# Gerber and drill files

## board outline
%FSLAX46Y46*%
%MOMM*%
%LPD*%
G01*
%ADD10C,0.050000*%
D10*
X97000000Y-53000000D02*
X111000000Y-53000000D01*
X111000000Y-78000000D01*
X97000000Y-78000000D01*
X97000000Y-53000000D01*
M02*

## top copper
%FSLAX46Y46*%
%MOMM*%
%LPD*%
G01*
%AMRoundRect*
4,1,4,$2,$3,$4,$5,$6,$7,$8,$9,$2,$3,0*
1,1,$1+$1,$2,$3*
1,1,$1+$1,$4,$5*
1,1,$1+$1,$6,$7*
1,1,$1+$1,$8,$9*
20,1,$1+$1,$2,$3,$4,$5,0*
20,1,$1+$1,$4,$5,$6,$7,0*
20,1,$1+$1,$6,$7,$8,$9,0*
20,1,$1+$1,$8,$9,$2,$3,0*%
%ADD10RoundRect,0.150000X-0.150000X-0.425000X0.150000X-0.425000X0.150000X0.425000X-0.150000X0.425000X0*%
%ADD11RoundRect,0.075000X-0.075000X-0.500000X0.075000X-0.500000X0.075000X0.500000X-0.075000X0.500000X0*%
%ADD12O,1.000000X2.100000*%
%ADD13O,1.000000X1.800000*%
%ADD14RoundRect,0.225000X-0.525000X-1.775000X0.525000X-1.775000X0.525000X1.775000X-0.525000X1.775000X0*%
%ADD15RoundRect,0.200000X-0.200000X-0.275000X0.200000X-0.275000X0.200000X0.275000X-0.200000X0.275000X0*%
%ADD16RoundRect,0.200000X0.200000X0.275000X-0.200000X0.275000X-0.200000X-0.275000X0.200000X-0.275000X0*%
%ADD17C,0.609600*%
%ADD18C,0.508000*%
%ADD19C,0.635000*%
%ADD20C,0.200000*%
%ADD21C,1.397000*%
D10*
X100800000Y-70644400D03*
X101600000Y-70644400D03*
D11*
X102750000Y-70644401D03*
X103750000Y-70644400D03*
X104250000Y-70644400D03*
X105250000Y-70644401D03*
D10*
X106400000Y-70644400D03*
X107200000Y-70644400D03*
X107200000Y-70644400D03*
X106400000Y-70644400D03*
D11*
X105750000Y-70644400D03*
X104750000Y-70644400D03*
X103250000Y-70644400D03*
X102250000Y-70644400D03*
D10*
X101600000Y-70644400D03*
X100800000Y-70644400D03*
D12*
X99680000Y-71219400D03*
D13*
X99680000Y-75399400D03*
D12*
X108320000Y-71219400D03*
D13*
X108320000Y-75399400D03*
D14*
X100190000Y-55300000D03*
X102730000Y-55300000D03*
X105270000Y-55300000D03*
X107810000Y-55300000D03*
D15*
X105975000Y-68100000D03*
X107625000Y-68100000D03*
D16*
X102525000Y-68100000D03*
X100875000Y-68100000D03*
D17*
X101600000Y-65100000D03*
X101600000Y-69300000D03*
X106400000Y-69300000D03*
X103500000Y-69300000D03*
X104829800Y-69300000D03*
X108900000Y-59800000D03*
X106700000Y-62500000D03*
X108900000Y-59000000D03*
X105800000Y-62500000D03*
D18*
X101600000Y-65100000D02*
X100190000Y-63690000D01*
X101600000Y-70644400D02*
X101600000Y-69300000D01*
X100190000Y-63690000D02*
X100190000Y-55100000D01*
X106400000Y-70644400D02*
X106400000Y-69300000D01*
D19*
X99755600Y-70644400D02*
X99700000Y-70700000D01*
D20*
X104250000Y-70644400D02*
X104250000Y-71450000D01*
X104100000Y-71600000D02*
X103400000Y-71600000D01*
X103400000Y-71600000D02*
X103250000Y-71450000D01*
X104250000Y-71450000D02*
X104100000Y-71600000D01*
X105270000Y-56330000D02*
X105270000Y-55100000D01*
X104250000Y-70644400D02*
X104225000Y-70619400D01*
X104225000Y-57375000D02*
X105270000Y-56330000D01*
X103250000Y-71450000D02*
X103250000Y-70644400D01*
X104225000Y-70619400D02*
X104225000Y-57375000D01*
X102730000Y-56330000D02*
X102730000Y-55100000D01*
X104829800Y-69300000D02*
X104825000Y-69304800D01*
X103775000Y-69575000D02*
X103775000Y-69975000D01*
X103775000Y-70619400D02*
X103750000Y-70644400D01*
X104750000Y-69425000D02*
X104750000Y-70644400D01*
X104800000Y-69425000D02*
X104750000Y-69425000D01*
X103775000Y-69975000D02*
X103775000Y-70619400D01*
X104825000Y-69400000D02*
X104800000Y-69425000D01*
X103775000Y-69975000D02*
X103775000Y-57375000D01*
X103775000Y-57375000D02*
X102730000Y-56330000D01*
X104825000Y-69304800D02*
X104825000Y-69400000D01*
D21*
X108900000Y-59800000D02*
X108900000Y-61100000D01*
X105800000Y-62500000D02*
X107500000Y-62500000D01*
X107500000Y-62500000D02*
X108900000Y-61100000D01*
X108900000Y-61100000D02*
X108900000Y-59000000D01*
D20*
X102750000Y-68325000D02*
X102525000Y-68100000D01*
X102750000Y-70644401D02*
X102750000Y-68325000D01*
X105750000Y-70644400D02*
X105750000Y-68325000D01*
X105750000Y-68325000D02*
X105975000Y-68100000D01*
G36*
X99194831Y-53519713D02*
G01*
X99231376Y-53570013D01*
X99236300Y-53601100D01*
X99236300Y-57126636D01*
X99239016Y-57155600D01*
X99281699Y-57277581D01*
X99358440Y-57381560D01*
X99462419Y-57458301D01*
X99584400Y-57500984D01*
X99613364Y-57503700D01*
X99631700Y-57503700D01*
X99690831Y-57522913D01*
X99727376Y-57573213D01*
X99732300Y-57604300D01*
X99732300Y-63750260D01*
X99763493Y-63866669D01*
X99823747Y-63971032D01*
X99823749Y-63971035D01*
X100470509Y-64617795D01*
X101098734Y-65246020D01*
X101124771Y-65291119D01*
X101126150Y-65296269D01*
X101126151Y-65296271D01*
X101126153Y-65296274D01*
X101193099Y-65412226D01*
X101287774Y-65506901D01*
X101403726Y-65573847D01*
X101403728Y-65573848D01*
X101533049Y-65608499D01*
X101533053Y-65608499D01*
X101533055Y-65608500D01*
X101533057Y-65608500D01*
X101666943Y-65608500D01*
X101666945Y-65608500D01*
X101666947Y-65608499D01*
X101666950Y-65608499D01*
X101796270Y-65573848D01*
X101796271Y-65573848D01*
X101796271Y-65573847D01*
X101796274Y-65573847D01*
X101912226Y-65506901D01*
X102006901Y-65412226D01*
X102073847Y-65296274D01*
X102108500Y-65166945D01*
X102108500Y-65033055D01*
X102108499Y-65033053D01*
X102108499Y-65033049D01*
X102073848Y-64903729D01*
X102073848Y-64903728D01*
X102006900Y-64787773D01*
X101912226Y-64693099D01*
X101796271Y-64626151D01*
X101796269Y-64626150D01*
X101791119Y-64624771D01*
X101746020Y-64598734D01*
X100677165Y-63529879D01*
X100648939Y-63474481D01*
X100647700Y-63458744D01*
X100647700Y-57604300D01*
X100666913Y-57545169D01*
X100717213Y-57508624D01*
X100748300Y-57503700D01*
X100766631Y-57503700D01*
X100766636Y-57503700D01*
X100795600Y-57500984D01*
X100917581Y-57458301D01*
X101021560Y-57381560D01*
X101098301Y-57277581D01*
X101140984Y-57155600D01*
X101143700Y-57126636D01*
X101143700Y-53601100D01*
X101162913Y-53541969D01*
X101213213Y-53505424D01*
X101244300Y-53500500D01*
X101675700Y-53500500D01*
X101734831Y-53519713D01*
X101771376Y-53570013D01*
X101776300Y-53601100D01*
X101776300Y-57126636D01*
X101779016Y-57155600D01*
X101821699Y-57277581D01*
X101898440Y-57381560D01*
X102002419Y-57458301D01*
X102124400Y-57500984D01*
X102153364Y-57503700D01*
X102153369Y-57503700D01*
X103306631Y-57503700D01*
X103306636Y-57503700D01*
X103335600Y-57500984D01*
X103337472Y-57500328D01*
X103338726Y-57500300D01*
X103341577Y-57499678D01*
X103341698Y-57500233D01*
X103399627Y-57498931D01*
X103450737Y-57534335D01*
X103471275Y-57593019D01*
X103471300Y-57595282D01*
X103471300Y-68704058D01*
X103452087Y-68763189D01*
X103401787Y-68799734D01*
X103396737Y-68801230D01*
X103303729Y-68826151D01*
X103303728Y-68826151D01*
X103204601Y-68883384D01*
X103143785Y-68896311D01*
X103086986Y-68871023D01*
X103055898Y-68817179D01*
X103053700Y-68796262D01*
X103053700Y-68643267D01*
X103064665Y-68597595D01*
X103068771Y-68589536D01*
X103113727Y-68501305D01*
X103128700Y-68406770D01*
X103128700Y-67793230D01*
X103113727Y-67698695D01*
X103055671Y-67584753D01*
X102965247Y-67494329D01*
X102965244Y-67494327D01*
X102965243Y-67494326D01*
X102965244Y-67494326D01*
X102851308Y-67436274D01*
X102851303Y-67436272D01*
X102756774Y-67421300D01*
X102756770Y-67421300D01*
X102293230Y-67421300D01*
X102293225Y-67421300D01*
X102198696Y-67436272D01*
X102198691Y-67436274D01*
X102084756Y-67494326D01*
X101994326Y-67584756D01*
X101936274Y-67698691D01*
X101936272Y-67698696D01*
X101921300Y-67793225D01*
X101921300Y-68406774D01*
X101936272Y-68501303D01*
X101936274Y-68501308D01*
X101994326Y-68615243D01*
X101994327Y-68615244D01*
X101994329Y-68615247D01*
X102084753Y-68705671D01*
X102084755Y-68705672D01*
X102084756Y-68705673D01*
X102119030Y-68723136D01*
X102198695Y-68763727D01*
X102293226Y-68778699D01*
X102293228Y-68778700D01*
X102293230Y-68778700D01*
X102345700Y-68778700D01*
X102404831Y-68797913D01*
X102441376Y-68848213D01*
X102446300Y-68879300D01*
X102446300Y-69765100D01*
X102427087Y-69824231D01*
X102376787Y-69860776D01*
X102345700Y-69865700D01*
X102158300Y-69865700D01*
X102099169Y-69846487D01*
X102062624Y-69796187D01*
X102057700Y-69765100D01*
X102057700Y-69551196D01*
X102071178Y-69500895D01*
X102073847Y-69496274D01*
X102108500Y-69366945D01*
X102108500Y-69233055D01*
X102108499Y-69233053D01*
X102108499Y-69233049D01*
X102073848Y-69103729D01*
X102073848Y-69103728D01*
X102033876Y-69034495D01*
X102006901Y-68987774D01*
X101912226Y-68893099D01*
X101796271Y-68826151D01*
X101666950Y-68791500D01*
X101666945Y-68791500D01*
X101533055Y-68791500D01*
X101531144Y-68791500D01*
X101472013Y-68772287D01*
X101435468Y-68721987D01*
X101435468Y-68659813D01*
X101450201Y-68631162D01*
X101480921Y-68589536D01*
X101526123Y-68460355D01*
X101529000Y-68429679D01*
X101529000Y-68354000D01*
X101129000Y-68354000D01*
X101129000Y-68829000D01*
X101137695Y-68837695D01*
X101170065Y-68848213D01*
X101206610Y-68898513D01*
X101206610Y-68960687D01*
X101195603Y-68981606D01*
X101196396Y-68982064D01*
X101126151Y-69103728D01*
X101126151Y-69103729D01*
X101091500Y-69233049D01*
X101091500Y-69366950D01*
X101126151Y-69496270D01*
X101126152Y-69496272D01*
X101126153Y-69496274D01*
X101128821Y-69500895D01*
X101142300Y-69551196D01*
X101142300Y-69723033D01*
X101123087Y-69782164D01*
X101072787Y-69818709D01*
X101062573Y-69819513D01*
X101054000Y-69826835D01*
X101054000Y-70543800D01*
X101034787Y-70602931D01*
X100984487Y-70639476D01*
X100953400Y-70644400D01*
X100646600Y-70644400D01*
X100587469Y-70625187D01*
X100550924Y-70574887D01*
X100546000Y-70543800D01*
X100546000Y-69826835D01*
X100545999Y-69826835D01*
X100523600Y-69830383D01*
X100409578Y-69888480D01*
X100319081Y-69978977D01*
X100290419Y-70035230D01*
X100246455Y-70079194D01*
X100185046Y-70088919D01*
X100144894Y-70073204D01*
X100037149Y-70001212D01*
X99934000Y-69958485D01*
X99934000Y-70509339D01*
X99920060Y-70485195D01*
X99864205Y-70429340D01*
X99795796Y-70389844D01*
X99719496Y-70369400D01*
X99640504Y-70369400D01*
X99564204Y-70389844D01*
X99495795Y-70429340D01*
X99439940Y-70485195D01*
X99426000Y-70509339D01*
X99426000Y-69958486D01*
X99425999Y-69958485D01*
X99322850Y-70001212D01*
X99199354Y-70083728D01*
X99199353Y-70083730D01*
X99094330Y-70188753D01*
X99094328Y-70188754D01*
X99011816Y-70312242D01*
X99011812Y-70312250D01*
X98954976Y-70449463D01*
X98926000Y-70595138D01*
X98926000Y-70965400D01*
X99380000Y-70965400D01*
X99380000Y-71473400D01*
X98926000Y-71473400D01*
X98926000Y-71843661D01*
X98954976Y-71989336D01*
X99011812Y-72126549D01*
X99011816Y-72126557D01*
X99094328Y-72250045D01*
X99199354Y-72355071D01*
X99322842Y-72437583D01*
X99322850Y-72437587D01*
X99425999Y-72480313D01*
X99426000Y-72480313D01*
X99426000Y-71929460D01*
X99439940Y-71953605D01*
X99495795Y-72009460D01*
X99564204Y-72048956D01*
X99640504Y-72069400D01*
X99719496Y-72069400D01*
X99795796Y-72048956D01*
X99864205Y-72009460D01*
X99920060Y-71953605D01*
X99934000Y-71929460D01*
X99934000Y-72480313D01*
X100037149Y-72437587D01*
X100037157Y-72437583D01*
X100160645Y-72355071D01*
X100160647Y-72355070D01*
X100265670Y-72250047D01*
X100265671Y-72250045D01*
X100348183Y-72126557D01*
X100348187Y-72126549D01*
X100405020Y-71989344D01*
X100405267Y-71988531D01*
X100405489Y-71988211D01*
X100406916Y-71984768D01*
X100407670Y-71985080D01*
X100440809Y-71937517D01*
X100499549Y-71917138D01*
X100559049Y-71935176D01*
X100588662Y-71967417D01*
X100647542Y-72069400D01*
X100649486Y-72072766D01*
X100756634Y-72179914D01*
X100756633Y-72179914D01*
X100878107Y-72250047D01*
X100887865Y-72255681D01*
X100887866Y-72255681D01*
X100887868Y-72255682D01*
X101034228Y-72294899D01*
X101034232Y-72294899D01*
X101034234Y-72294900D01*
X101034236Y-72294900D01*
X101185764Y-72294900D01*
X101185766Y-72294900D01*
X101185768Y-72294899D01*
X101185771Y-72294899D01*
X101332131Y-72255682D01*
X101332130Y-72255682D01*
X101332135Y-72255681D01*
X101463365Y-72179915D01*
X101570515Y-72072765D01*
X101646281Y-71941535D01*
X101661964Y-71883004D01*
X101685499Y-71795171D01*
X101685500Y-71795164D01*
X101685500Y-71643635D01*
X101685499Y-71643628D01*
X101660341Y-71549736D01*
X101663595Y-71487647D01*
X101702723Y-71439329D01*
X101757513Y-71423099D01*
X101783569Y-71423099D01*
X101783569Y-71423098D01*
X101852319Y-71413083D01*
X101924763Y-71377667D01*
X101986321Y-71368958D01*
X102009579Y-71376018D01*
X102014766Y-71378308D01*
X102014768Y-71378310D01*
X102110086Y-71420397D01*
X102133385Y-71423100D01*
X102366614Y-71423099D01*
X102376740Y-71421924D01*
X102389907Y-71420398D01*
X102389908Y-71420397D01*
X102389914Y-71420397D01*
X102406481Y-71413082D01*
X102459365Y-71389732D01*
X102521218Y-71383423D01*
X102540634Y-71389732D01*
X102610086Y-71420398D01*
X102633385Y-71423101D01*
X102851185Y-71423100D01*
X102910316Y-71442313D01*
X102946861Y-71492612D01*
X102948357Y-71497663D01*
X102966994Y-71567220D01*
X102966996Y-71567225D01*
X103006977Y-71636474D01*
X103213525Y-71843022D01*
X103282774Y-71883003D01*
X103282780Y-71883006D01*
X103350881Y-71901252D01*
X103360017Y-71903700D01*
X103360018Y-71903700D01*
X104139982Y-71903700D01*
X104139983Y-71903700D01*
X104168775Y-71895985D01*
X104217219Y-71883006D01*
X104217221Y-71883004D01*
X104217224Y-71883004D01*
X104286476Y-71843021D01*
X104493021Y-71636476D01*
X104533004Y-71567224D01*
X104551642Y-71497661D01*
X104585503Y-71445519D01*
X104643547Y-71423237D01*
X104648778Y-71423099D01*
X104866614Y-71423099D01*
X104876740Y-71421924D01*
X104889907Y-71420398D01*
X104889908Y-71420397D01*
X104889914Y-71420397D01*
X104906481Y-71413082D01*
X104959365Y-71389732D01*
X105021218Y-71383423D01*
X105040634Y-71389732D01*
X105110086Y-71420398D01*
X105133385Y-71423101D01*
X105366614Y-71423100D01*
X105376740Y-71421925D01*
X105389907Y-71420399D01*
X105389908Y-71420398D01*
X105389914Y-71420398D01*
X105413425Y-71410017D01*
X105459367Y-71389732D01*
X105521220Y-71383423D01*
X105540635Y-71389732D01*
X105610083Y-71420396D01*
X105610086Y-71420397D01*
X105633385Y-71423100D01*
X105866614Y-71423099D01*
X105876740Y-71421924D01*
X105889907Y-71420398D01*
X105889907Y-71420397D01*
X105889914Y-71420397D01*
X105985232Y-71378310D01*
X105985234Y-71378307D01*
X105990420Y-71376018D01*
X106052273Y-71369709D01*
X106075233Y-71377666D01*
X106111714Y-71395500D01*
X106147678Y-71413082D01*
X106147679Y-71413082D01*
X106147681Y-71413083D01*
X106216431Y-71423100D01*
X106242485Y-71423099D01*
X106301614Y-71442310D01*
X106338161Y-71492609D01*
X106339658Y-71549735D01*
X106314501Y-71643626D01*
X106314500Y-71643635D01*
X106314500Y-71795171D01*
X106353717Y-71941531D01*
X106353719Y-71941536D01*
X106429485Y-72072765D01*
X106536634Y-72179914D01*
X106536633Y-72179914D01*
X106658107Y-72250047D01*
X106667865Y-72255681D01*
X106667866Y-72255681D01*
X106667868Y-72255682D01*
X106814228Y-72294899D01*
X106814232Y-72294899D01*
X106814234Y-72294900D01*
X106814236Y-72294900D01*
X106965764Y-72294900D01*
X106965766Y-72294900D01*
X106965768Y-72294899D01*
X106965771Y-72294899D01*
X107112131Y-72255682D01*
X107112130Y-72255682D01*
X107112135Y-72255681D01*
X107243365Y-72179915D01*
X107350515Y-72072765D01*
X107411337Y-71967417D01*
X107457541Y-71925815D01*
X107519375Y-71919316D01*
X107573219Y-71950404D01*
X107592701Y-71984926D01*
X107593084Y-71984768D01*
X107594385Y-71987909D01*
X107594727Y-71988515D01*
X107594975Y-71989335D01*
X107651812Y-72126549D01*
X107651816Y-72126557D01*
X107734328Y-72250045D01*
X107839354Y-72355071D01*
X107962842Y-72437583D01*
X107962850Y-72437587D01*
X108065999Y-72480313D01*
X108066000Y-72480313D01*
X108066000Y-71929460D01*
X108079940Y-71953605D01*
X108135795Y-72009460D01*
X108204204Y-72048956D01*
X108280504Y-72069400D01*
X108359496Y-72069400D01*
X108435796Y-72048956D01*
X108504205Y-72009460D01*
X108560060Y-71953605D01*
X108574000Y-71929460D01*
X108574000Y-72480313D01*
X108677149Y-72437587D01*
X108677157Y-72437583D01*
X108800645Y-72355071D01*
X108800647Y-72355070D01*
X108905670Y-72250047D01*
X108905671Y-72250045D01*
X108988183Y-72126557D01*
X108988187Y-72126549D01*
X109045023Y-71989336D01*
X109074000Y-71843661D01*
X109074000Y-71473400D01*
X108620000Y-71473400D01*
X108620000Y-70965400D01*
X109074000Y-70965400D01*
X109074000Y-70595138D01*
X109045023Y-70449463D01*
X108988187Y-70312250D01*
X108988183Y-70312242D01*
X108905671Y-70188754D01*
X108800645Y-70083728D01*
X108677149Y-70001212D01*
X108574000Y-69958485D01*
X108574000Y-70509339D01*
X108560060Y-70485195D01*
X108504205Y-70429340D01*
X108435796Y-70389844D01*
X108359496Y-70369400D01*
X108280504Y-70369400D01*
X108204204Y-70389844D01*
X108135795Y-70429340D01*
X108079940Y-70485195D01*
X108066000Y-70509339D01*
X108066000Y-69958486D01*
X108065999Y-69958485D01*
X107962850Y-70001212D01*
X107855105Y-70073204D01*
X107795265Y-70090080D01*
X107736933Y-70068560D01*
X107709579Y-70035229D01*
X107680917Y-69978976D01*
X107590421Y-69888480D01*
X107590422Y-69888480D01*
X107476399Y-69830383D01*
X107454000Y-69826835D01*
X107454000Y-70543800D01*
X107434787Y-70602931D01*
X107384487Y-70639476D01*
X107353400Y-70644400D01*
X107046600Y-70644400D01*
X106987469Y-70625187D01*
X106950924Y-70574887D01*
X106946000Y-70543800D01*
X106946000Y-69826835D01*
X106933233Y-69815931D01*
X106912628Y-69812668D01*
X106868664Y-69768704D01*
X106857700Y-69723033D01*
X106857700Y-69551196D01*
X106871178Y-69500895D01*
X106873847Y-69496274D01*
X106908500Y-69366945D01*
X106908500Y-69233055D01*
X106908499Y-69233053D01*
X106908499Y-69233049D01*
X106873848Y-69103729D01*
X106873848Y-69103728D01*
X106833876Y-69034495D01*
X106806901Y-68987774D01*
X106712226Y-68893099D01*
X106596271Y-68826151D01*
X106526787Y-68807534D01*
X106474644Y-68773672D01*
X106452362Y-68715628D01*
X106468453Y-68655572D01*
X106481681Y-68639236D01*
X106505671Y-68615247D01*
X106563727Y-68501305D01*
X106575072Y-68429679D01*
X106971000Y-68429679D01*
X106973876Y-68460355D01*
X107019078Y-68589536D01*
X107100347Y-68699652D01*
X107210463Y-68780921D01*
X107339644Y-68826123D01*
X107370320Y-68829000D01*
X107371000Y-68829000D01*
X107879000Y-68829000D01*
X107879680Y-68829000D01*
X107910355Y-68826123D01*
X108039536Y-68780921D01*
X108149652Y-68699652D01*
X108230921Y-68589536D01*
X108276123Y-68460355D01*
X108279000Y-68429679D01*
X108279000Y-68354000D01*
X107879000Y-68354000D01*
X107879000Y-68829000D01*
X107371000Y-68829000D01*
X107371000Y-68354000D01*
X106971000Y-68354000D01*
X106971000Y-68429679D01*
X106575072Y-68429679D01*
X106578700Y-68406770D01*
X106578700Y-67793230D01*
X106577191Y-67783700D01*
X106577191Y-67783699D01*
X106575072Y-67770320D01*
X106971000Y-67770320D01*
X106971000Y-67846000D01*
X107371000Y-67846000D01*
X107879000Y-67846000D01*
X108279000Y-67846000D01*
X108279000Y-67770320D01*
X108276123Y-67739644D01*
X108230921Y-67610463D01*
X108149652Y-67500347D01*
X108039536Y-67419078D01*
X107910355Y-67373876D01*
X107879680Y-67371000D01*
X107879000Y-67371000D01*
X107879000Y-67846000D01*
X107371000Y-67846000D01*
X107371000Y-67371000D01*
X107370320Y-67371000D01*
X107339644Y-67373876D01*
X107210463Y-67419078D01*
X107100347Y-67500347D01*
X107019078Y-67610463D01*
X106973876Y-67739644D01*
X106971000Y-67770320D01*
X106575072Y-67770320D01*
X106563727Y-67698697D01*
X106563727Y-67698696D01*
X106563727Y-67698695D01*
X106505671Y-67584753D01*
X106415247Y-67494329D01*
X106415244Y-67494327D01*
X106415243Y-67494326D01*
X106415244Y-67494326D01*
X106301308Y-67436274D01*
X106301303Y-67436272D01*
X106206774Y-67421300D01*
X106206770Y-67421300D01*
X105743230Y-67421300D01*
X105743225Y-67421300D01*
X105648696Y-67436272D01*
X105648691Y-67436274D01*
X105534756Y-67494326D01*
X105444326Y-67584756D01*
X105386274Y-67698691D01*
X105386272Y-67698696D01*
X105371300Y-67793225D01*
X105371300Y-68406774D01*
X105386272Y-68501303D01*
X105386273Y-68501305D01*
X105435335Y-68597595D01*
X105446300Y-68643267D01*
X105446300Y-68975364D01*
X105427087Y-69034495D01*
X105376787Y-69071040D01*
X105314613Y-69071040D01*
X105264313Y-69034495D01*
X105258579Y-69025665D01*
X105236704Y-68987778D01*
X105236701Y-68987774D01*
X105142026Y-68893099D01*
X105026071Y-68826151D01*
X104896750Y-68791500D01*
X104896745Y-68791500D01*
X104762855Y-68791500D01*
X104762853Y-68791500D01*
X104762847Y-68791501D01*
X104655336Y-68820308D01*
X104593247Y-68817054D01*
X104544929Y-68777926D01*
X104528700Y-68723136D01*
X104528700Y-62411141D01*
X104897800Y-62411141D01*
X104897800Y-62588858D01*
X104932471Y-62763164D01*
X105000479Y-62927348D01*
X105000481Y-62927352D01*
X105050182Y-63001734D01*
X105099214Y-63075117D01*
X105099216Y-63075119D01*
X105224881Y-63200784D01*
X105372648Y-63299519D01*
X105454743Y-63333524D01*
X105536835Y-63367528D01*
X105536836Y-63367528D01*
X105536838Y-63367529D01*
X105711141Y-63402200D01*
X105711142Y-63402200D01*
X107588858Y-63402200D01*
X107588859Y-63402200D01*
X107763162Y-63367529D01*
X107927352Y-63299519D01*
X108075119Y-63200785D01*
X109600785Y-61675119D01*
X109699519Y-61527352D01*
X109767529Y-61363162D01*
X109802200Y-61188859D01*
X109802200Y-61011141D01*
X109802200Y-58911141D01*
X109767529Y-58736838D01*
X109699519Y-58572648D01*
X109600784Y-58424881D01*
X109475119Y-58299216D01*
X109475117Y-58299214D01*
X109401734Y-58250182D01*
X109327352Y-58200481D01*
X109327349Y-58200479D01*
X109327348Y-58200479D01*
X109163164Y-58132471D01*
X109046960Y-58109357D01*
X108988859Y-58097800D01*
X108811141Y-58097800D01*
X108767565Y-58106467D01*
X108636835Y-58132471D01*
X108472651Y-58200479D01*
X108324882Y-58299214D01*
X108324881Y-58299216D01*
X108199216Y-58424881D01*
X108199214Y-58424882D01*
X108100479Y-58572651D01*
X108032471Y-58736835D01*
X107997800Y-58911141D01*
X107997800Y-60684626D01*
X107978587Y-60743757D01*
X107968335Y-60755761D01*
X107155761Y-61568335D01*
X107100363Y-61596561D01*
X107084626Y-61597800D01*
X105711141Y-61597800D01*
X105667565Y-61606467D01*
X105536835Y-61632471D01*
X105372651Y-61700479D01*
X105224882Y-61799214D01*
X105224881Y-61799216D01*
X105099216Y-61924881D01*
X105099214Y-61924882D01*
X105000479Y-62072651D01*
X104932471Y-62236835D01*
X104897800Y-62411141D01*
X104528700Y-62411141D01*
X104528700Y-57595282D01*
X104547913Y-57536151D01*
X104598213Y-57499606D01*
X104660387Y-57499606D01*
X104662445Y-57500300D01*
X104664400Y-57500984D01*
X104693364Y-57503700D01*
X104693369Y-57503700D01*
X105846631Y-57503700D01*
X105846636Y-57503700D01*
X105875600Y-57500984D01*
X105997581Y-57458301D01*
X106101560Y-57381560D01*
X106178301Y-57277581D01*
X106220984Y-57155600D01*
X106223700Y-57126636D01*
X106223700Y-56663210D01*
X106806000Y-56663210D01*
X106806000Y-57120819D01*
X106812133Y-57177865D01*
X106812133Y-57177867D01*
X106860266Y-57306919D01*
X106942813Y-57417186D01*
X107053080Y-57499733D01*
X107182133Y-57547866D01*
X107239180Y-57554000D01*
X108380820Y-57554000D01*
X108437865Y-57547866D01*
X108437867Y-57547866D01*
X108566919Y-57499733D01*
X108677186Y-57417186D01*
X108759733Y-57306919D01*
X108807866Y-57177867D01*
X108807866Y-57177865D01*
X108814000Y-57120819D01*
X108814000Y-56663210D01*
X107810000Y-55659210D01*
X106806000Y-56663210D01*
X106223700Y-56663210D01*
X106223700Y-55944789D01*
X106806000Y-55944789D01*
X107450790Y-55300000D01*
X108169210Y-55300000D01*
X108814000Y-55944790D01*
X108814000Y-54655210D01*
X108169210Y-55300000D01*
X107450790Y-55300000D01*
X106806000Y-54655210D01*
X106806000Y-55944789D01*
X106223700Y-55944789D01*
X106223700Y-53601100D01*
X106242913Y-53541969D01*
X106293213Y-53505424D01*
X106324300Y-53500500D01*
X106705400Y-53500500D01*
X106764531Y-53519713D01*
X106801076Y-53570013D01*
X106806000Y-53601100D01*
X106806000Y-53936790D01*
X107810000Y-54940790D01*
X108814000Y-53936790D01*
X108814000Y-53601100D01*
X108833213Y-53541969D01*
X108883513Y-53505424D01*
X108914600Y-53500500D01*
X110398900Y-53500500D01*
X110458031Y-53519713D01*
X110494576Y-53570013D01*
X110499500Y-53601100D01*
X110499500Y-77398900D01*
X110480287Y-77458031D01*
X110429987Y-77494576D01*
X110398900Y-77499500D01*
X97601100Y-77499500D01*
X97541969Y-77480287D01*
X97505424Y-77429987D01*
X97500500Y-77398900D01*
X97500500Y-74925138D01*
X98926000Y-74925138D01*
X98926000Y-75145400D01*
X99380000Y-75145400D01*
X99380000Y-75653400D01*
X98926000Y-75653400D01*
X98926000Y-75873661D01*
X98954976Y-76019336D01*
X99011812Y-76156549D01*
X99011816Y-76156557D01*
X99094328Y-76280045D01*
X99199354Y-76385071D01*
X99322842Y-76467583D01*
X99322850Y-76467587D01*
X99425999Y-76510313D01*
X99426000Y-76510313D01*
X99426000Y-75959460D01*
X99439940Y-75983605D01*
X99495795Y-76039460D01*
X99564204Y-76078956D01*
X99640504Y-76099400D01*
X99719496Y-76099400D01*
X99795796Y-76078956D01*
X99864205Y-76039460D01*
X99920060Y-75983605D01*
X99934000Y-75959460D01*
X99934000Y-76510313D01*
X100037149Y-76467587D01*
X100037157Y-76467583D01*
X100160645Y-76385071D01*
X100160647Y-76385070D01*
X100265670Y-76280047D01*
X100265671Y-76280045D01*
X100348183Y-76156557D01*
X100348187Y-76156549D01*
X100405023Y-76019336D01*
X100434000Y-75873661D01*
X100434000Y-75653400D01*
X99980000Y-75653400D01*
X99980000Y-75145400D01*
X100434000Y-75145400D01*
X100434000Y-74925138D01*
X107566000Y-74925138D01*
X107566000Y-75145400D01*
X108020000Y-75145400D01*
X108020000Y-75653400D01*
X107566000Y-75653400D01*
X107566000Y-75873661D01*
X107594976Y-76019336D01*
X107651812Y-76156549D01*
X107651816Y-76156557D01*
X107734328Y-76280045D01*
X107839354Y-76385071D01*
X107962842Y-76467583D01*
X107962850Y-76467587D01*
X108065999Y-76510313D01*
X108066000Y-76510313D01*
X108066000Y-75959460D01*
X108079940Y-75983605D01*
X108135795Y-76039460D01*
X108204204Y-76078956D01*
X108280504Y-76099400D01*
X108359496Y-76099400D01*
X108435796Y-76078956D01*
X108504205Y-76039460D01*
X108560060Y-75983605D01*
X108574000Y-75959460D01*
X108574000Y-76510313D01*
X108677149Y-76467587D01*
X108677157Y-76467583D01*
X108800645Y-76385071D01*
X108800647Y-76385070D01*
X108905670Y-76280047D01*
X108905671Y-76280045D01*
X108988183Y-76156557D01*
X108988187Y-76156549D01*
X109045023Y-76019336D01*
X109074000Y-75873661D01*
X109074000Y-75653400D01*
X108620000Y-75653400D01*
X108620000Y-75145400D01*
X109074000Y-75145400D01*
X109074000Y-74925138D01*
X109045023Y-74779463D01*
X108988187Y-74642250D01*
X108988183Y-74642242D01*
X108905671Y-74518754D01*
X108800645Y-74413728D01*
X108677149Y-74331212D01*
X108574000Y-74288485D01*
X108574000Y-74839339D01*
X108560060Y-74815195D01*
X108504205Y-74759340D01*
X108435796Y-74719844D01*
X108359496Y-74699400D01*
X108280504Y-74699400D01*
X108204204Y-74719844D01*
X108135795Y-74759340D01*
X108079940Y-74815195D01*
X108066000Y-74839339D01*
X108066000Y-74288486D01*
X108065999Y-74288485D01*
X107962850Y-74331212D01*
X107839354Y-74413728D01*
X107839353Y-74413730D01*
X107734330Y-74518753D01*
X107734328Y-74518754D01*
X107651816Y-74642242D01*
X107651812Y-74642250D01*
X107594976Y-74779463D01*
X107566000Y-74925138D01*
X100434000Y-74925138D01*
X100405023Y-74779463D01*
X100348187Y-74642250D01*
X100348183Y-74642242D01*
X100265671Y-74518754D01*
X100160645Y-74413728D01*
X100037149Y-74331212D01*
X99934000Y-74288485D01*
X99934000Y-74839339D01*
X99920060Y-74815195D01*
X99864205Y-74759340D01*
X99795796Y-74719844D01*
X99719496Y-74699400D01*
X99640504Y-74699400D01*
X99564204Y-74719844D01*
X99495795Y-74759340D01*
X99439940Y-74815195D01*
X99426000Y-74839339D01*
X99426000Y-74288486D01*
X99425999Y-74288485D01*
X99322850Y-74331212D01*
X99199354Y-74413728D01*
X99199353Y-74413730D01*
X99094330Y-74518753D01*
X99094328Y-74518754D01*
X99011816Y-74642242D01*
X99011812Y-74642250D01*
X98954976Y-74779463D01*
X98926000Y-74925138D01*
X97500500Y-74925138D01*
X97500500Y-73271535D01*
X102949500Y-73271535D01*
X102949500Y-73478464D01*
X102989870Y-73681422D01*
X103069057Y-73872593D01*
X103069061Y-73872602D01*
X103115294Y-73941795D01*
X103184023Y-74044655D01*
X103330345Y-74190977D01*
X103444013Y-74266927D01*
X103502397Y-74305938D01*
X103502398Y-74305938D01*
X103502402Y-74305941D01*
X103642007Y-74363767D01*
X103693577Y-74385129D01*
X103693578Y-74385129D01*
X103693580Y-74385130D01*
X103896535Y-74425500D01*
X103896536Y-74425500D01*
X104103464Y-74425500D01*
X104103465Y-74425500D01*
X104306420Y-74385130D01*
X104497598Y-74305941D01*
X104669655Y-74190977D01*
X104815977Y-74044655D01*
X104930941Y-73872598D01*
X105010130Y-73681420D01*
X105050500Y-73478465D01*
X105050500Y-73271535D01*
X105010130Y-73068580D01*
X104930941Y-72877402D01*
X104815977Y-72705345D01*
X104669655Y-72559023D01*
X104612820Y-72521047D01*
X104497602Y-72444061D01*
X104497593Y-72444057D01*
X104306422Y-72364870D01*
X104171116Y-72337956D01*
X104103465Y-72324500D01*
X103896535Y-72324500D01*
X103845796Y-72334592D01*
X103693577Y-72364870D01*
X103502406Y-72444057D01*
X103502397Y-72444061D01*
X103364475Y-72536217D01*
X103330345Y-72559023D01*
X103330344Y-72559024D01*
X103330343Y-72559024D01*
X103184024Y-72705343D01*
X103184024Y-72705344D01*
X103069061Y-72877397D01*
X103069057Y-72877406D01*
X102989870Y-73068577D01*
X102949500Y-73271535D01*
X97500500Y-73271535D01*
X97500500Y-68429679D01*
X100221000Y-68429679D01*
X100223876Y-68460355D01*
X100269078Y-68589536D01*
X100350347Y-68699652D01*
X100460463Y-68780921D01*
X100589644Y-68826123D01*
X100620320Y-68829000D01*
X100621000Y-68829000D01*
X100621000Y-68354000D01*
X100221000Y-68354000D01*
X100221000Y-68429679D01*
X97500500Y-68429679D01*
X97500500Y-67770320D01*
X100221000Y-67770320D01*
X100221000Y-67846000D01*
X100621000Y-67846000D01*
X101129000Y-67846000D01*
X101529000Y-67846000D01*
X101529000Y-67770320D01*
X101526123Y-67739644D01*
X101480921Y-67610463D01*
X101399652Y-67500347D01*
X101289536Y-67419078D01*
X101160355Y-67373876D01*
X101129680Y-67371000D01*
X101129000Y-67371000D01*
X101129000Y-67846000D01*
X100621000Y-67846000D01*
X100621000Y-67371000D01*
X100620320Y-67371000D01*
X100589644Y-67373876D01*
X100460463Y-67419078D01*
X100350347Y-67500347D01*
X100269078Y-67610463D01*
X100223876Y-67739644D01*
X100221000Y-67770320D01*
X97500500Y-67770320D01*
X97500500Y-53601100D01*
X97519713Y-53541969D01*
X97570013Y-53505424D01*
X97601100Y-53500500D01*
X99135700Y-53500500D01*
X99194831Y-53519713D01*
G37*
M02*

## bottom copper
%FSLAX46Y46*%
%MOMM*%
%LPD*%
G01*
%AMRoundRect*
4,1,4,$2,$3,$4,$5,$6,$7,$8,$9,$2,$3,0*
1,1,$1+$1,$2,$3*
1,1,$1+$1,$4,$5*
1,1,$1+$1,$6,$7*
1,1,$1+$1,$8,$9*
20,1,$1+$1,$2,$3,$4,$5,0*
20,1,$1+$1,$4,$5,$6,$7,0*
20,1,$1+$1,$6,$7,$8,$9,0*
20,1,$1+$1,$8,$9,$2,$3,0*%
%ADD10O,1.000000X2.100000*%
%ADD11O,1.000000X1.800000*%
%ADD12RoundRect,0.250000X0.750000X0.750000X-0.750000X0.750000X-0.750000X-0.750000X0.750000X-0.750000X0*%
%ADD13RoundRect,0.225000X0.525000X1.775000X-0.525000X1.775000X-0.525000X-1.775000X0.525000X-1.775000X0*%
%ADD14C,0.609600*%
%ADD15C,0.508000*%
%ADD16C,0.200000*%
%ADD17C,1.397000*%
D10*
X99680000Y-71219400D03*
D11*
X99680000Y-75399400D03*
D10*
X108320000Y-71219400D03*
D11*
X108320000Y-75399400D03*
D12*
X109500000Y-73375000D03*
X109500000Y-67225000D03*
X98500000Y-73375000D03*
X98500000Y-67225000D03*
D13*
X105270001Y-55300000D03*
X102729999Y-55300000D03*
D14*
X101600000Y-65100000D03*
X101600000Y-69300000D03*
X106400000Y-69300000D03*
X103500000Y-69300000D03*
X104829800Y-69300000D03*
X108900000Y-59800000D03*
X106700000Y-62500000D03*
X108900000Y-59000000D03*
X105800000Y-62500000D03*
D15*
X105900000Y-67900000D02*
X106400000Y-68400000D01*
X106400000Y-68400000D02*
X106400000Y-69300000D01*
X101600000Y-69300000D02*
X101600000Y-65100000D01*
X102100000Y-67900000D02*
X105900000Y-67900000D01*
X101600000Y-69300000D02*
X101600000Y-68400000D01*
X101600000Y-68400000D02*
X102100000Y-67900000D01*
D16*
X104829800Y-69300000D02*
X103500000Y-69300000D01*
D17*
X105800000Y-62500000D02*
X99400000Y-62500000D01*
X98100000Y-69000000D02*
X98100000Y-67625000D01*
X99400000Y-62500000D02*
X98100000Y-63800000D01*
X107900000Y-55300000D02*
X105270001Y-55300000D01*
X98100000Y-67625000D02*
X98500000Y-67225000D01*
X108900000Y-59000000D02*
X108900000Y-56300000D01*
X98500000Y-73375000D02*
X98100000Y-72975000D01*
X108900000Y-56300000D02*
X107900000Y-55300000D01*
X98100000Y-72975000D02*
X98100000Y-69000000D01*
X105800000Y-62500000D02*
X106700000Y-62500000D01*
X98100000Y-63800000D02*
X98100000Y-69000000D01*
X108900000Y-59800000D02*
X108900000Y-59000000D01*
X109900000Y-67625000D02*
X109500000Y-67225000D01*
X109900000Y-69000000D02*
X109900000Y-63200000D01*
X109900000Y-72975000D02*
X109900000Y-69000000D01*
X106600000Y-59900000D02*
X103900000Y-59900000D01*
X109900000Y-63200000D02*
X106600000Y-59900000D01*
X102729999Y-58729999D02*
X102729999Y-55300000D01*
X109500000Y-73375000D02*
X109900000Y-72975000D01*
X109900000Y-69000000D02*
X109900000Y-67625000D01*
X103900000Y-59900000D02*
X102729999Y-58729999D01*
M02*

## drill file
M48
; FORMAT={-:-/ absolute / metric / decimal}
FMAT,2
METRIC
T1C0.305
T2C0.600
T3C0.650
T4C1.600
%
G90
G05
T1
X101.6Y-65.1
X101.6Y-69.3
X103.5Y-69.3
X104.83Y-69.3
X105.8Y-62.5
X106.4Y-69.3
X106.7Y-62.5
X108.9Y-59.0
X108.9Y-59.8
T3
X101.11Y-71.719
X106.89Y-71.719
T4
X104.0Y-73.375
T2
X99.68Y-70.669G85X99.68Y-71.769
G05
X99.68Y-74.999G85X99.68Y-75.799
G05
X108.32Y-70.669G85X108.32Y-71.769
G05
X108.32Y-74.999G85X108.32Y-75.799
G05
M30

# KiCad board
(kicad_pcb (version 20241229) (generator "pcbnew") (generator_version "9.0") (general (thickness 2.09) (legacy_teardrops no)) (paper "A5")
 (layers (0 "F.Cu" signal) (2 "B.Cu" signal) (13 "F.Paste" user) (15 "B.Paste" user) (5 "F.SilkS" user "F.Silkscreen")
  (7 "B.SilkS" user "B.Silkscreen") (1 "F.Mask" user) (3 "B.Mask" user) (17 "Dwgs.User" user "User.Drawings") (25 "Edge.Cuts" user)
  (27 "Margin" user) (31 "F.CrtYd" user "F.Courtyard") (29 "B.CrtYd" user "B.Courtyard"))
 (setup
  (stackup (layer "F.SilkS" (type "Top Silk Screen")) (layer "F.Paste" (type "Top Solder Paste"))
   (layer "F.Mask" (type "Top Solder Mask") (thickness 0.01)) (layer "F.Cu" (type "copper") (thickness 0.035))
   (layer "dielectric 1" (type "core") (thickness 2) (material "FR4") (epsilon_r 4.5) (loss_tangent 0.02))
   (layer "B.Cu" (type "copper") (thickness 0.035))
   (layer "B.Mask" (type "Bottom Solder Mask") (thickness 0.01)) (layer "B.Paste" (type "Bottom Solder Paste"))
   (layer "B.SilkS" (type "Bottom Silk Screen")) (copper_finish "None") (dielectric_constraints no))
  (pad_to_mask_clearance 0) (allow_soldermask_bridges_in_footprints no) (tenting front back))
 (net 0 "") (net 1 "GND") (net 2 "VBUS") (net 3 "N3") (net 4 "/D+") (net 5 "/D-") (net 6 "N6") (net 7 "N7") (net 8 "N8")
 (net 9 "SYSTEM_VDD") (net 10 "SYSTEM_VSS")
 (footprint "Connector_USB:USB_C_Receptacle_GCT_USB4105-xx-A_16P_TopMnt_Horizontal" (layer "F.Cu") (at 104 74.3244)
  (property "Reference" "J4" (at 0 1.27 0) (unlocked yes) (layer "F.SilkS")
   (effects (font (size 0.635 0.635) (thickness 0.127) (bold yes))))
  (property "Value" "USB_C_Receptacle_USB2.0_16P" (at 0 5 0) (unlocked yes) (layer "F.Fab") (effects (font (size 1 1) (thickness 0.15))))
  (pad "" np_thru_hole circle (at -2.89 -2.605) (size 0.65 0.65) (drill 0.65) (layers "*.Cu" "*.Mask"))
  (pad "" np_thru_hole circle (at 2.89 -2.605) (size 0.65 0.65) (drill 0.65) (layers "*.Cu" "*.Mask"))
  (pad "A1" smd roundrect (at -3.2 -3.68) (size 0.6 1.15) (layers "F.Cu" "F.Mask" "F.Paste") (roundrect_rratio 0.25) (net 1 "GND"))
  (pad "A4" smd roundrect (at -2.4 -3.68) (size 0.6 1.15) (layers "F.Cu" "F.Mask" "F.Paste") (roundrect_rratio 0.25) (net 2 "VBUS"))
  (pad "A5" smd roundrect (at -1.25 -3.679999) (size 0.3 1.15) (layers "F.Cu" "F.Mask" "F.Paste") (roundrect_rratio 0.25) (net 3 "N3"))
  (pad "A6" smd roundrect (at -0.25 -3.68) (size 0.3 1.15) (layers "F.Cu" "F.Mask" "F.Paste") (roundrect_rratio 0.25) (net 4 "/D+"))
  (pad "A7" smd roundrect (at 0.25 -3.68) (size 0.3 1.15) (layers "F.Cu" "F.Mask" "F.Paste") (roundrect_rratio 0.25) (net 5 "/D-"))
  (pad "A8" smd roundrect (at 1.25 -3.679999) (size 0.3 1.15) (layers "F.Cu" "F.Mask" "F.Paste") (roundrect_rratio 0.25) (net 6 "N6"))
  (pad "A9" smd roundrect (at 2.4 -3.68) (size 0.6 1.15) (layers "F.Cu" "F.Mask" "F.Paste") (roundrect_rratio 0.25) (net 2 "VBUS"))
  (pad "A12" smd roundrect (at 3.2 -3.68) (size 0.6 1.15) (layers "F.Cu" "F.Mask" "F.Paste") (roundrect_rratio 0.25) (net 1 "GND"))
  (pad "B1" smd roundrect (at 3.2 -3.68) (size 0.6 1.15) (layers "F.Cu" "F.Mask" "F.Paste") (roundrect_rratio 0.25) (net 1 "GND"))
  (pad "B4" smd roundrect (at 2.4 -3.68) (size 0.6 1.15) (layers "F.Cu" "F.Mask" "F.Paste") (roundrect_rratio 0.25) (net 2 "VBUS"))
  (pad "B5" smd roundrect (at 1.75 -3.68) (size 0.3 1.15) (layers "F.Cu" "F.Mask" "F.Paste") (roundrect_rratio 0.25) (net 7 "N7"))
  (pad "B6" smd roundrect (at 0.75 -3.68) (size 0.3 1.15) (layers "F.Cu" "F.Mask" "F.Paste") (roundrect_rratio 0.25) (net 4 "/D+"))
  (pad "B7" smd roundrect (at -0.75 -3.68) (size 0.3 1.15) (layers "F.Cu" "F.Mask" "F.Paste") (roundrect_rratio 0.25) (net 5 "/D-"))
  (pad "B8" smd roundrect (at -1.75 -3.68) (size 0.3 1.15) (layers "F.Cu" "F.Mask" "F.Paste") (roundrect_rratio 0.25) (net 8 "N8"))
  (pad "B9" smd roundrect (at -2.4 -3.68) (size 0.6 1.15) (layers "F.Cu" "F.Mask" "F.Paste") (roundrect_rratio 0.25) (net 2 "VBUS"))
  (pad "B12" smd roundrect (at -3.2 -3.68) (size 0.6 1.15) (layers "F.Cu" "F.Mask" "F.Paste") (roundrect_rratio 0.25) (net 1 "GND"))
  (pad "S1" thru_hole oval (at -4.32 -3.105) (size 1 2.1) (drill oval 0.6 1.7) (layers "*.Cu" "*.Mask" "F.Paste") (remove_unused_layers no)
   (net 1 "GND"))
  (pad "S1" thru_hole oval (at -4.32 1.075) (size 1 1.8) (drill oval 0.6 1.4) (layers "*.Cu" "*.Mask" "F.Paste") (remove_unused_layers no)
   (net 1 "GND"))
  (pad "S1" thru_hole oval (at 4.32 -3.105) (size 1 2.1) (drill oval 0.6 1.7) (layers "*.Cu" "*.Mask" "F.Paste") (remove_unused_layers no)
   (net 1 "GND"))
  (pad "S1" thru_hole oval (at 4.32 1.075) (size 1 1.8) (drill oval 0.6 1.4) (layers "*.Cu" "*.Mask" "F.Paste") (remove_unused_layers no)
   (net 1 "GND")))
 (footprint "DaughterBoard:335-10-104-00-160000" (layer "F.Cu") (at 104 55.3)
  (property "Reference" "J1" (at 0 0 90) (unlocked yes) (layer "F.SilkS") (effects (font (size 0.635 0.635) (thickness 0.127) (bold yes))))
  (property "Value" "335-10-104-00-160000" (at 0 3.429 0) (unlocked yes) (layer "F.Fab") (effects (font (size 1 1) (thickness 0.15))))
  (pad "1" smd roundrect (at -3.81 0) (size 1.5 4) (layers "F.Cu" "F.Mask" "F.Paste") (roundrect_rratio 0.15) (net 2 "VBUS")
   (thermal_bridge_angle 45))
  (pad "2" smd roundrect (at -1.27 0) (size 1.5 4) (layers "F.Cu" "F.Mask" "F.Paste") (roundrect_rratio 0.15) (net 4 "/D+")
   (thermal_bridge_angle 45))
  (pad "3" smd roundrect (at 1.27 0) (size 1.5 4) (layers "F.Cu" "F.Mask" "F.Paste") (roundrect_rratio 0.15) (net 5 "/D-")
   (thermal_bridge_angle 45))
  (pad "4" smd roundrect (at 3.81 0) (size 1.5 4) (layers "F.Cu" "F.Mask" "F.Paste") (roundrect_rratio 0.15) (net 1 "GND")
   (thermal_bridge_angle 45)))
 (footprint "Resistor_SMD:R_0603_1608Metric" (layer "F.Cu") (at 106.8 68.1)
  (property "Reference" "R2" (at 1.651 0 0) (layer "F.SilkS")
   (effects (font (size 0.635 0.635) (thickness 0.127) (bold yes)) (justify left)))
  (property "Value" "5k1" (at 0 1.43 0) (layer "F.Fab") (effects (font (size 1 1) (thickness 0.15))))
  (pad "1" smd roundrect (at -0.825 0) (size 0.8 0.95) (layers "F.Cu" "F.Mask" "F.Paste") (roundrect_rratio 0.25) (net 7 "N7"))
  (pad "2" smd roundrect (at 0.825 0) (size 0.8 0.95) (layers "F.Cu" "F.Mask" "F.Paste") (roundrect_rratio 0.25) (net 1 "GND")))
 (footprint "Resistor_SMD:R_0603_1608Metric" (layer "F.Cu") (at 101.7 68.1 180)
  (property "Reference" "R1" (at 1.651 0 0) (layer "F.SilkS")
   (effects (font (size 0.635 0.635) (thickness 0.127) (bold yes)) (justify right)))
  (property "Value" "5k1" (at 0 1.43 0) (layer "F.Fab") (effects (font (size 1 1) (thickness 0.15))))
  (pad "1" smd roundrect (at -0.825 0 180) (size 0.8 0.95) (layers "F.Cu" "F.Mask" "F.Paste") (roundrect_rratio 0.25) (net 3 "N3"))
  (pad "2" smd roundrect (at 0.825 0 180) (size 0.8 0.95) (layers "F.Cu" "F.Mask" "F.Paste") (roundrect_rratio 0.25) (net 1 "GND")))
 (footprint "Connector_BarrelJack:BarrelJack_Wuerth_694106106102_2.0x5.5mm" (layer "B.Cu") (at 104 70.3 180)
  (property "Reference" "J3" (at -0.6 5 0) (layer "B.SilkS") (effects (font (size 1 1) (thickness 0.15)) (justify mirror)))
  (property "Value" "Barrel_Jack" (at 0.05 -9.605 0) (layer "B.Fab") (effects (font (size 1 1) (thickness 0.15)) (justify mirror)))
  (pad "" np_thru_hole circle (at 0 -3.075 180) (size 1.6 1.6) (drill 1.6) (layers "*.Cu" "*.Mask"))
  (pad "1" smd roundrect (at -5.5 -3.075 180) (size 2 2) (layers "B.Cu" "B.Mask" "B.Paste") (roundrect_rratio 0.125) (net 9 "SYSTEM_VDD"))
  (pad "1" smd roundrect (at -5.5 3.075 180) (size 2 2) (layers "B.Cu" "B.Mask" "B.Paste") (roundrect_rratio 0.125) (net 9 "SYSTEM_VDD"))
  (pad "2" smd roundrect (at 5.5 -3.075 180) (size 2 2) (layers "B.Cu" "B.Mask" "B.Paste") (roundrect_rratio 0.125) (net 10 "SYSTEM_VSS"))
  (pad "3" smd roundrect (at 5.5 3.075 180) (size 2 2) (layers "B.Cu" "B.Mask" "B.Paste") (roundrect_rratio 0.125) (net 10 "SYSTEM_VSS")))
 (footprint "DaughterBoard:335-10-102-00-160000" (layer "B.Cu") (at 104 55.3 180)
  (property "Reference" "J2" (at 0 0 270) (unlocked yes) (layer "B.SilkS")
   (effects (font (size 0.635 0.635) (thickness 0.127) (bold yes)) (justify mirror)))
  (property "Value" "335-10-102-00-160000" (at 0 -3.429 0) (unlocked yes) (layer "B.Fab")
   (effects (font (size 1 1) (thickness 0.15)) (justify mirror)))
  (pad "1" smd roundrect (at -1.270001 0 180) (size 1.5 4) (layers "B.Cu" "B.Mask" "B.Paste") (roundrect_rratio 0.15) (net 10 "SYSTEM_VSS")
   (thermal_bridge_angle 45))
  (pad "2" smd roundrect (at 1.270001 0 180) (size 1.5 4) (layers "B.Cu" "B.Mask" "B.Paste") (roundrect_rratio 0.15) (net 9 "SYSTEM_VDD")
   (thermal_bridge_angle 45)))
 (gr_rect (start 97 53) (end 111 78) (stroke (width 0.05) (type solid)) (fill no) (layer "Edge.Cuts"))
 (segment (start 101.6 65.1) (end 100.19 63.69) (width 0.508) (layer "F.Cu") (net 2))
 (segment (start 101.6 70.6444) (end 101.6 69.3) (width 0.508) (layer "F.Cu") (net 2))
 (segment (start 100.19 63.69) (end 100.19 55.1) (width 0.508) (layer "F.Cu") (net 2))
 (segment (start 106.4 70.6444) (end 106.4 69.3) (width 0.508) (layer "F.Cu") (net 2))
 (via (at 101.6 65.1) (size 0.6096) (drill 0.3048) (layers "F.Cu" "B.Cu") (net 2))
 (via (at 101.6 69.3) (size 0.6096) (drill 0.3048) (layers "F.Cu" "B.Cu") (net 2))
 (via (at 106.4 69.3) (size 0.6096) (drill 0.3048) (layers "F.Cu" "B.Cu") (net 2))
 (segment (start 105.9 67.9) (end 106.4 68.4) (width 0.508) (layer "B.Cu") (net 2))
 (segment (start 106.4 68.4) (end 106.4 69.3) (width 0.508) (layer "B.Cu") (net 2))
 (segment (start 101.6 69.3) (end 101.6 65.1) (width 0.508) (layer "B.Cu") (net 2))
 (segment (start 102.1 67.9) (end 105.9 67.9) (width 0.508) (layer "B.Cu") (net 2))
 (segment (start 101.6 69.3) (end 101.6 68.4) (width 0.508) (layer "B.Cu") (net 2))
 (segment (start 101.6 68.4) (end 102.1 67.9) (width 0.508) (layer "B.Cu") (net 2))
 (segment (start 99.7556 70.6444) (end 99.7 70.7) (width 0.635) (layer "F.Cu") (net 1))
 (segment (start 104.25 70.6444) (end 104.25 71.45) (width 0.2) (layer "F.Cu") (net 5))
 (segment (start 104.1 71.6) (end 103.4 71.6) (width 0.2) (layer "F.Cu") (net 5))
 (segment (start 103.4 71.6) (end 103.25 71.45) (width 0.2) (layer "F.Cu") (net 5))
 (segment (start 104.25 71.45) (end 104.1 71.6) (width 0.2) (layer "F.Cu") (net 5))
 (segment (start 105.27 56.33) (end 105.27 55.1) (width 0.2) (layer "F.Cu") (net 5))
 (segment (start 104.25 70.6444) (end 104.225 70.6194) (width 0.2) (layer "F.Cu") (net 5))
 (segment (start 104.225 57.375) (end 105.27 56.33) (width 0.2) (layer "F.Cu") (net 5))
 (segment (start 103.25 71.45) (end 103.25 70.6444) (width 0.2) (layer "F.Cu") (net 5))
 (segment (start 104.225 70.6194) (end 104.225 57.375) (width 0.2) (layer "F.Cu") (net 5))
 (segment (start 102.73 56.33) (end 102.73 55.1) (width 0.2) (layer "F.Cu") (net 4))
 (segment (start 104.8298 69.3) (end 104.825 69.3048) (width 0.2) (layer "F.Cu") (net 4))
 (segment (start 103.775 69.575) (end 103.775 69.975) (width 0.2) (layer "F.Cu") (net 4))
 (segment (start 103.775 70.6194) (end 103.75 70.6444) (width 0.2) (layer "F.Cu") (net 4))
 (segment (start 104.75 69.425) (end 104.75 70.6444) (width 0.2) (layer "F.Cu") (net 4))
 (segment (start 104.8 69.425) (end 104.75 69.425) (width 0.2) (layer "F.Cu") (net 4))
 (segment (start 103.775 69.975) (end 103.775 70.6194) (width 0.2) (layer "F.Cu") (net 4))
 (segment (start 104.825 69.4) (end 104.8 69.425) (width 0.2) (layer "F.Cu") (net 4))
 (segment (start 103.775 69.975) (end 103.775 57.375) (width 0.2) (layer "F.Cu") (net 4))
 (segment (start 103.775 57.375) (end 102.73 56.33) (width 0.2) (layer "F.Cu") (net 4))
 (segment (start 104.825 69.3048) (end 104.825 69.4) (width 0.2) (layer "F.Cu") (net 4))
 (via (at 103.5 69.3) (size 0.6096) (drill 0.3048) (layers "F.Cu" "B.Cu") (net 4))
 (via (at 104.8298 69.3) (size 0.6096) (drill 0.3048) (layers "F.Cu" "B.Cu") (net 4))
 (segment (start 104.8298 69.3) (end 103.5 69.3) (width 0.2) (layer "B.Cu") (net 4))
 (segment (start 108.9 59.8) (end 108.9 61.1) (width 1.397) (layer "F.Cu") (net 10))
 (segment (start 105.8 62.5) (end 107.5 62.5) (width 1.397) (layer "F.Cu") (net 10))
 (segment (start 107.5 62.5) (end 108.9 61.1) (width 1.397) (layer "F.Cu") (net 10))
 (segment (start 108.9 61.1) (end 108.9 59) (width 1.397) (layer "F.Cu") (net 10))
 (via (at 108.9 59.8) (size 0.6096) (drill 0.3048) (layers "F.Cu" "B.Cu") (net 10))
 (via (at 106.7 62.5) (size 0.6096) (drill 0.3048) (layers "F.Cu" "B.Cu") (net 10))
 (via (at 108.9 59) (size 0.6096) (drill 0.3048) (layers "F.Cu" "B.Cu") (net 10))
 (via (at 105.8 62.5) (size 0.6096) (drill 0.3048) (layers "F.Cu" "B.Cu") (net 10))
 (segment (start 105.8 62.5) (end 99.4 62.5) (width 1.397) (layer "B.Cu") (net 10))
 (segment (start 98.1 69) (end 98.1 67.625) (width 1.397) (layer "B.Cu") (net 10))
 (segment (start 99.4 62.5) (end 98.1 63.8) (width 1.397) (layer "B.Cu") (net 10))
 (segment (start 107.9 55.3) (end 105.270001 55.3) (width 1.397) (layer "B.Cu") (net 10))
 (segment (start 98.1 67.625) (end 98.5 67.225) (width 1.397) (layer "B.Cu") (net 10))
 (segment (start 108.9 59) (end 108.9 56.3) (width 1.397) (layer "B.Cu") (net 10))
 (segment (start 98.5 73.375) (end 98.1 72.975) (width 1.397) (layer "B.Cu") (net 10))
 (segment (start 108.9 56.3) (end 107.9 55.3) (width 1.397) (layer "B.Cu") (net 10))
 (segment (start 98.1 72.975) (end 98.1 69) (width 1.397) (layer "B.Cu") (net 10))
 (segment (start 105.8 62.5) (end 106.7 62.5) (width 1.397) (layer "B.Cu") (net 10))
 (segment (start 98.1 63.8) (end 98.1 69) (width 1.397) (layer "B.Cu") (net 10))
 (segment (start 108.9 59.8) (end 108.9 59) (width 1.397) (layer "B.Cu") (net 10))
 (segment (start 109.9 67.625) (end 109.5 67.225) (width 1.397) (layer "B.Cu") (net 9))
 (segment (start 109.9 69) (end 109.9 63.2) (width 1.397) (layer "B.Cu") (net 9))
 (segment (start 109.9 72.975) (end 109.9 69) (width 1.397) (layer "B.Cu") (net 9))
 (segment (start 106.6 59.9) (end 103.9 59.9) (width 1.397) (layer "B.Cu") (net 9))
 (segment (start 109.9 63.2) (end 106.6 59.9) (width 1.397) (layer "B.Cu") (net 9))
 (segment (start 102.729999 58.729999) (end 102.729999 55.3) (width 1.397) (layer "B.Cu") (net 9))
 (segment (start 109.5 73.375) (end 109.9 72.975) (width 1.397) (layer "B.Cu") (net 9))
 (segment (start 109.9 69) (end 109.9 67.625) (width 1.397) (layer "B.Cu") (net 9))
 (segment (start 103.9 59.9) (end 102.729999 58.729999) (width 1.397) (layer "B.Cu") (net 9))
 (segment (start 102.75 68.325) (end 102.525 68.1) (width 0.2) (layer "F.Cu") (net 3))
 (segment (start 102.75 70.644401) (end 102.75 68.325) (width 0.2) (layer "F.Cu") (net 3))
 (segment (start 105.75 70.6444) (end 105.75 68.325) (width 0.2) (layer "F.Cu") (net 7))
 (segment (start 105.75 68.325) (end 105.975 68.1) (width 0.2) (layer "F.Cu") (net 7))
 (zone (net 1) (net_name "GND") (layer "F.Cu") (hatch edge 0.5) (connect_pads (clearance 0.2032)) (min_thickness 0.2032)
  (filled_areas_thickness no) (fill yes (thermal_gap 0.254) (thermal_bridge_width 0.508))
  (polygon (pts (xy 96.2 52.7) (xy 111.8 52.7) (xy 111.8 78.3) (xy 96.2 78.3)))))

